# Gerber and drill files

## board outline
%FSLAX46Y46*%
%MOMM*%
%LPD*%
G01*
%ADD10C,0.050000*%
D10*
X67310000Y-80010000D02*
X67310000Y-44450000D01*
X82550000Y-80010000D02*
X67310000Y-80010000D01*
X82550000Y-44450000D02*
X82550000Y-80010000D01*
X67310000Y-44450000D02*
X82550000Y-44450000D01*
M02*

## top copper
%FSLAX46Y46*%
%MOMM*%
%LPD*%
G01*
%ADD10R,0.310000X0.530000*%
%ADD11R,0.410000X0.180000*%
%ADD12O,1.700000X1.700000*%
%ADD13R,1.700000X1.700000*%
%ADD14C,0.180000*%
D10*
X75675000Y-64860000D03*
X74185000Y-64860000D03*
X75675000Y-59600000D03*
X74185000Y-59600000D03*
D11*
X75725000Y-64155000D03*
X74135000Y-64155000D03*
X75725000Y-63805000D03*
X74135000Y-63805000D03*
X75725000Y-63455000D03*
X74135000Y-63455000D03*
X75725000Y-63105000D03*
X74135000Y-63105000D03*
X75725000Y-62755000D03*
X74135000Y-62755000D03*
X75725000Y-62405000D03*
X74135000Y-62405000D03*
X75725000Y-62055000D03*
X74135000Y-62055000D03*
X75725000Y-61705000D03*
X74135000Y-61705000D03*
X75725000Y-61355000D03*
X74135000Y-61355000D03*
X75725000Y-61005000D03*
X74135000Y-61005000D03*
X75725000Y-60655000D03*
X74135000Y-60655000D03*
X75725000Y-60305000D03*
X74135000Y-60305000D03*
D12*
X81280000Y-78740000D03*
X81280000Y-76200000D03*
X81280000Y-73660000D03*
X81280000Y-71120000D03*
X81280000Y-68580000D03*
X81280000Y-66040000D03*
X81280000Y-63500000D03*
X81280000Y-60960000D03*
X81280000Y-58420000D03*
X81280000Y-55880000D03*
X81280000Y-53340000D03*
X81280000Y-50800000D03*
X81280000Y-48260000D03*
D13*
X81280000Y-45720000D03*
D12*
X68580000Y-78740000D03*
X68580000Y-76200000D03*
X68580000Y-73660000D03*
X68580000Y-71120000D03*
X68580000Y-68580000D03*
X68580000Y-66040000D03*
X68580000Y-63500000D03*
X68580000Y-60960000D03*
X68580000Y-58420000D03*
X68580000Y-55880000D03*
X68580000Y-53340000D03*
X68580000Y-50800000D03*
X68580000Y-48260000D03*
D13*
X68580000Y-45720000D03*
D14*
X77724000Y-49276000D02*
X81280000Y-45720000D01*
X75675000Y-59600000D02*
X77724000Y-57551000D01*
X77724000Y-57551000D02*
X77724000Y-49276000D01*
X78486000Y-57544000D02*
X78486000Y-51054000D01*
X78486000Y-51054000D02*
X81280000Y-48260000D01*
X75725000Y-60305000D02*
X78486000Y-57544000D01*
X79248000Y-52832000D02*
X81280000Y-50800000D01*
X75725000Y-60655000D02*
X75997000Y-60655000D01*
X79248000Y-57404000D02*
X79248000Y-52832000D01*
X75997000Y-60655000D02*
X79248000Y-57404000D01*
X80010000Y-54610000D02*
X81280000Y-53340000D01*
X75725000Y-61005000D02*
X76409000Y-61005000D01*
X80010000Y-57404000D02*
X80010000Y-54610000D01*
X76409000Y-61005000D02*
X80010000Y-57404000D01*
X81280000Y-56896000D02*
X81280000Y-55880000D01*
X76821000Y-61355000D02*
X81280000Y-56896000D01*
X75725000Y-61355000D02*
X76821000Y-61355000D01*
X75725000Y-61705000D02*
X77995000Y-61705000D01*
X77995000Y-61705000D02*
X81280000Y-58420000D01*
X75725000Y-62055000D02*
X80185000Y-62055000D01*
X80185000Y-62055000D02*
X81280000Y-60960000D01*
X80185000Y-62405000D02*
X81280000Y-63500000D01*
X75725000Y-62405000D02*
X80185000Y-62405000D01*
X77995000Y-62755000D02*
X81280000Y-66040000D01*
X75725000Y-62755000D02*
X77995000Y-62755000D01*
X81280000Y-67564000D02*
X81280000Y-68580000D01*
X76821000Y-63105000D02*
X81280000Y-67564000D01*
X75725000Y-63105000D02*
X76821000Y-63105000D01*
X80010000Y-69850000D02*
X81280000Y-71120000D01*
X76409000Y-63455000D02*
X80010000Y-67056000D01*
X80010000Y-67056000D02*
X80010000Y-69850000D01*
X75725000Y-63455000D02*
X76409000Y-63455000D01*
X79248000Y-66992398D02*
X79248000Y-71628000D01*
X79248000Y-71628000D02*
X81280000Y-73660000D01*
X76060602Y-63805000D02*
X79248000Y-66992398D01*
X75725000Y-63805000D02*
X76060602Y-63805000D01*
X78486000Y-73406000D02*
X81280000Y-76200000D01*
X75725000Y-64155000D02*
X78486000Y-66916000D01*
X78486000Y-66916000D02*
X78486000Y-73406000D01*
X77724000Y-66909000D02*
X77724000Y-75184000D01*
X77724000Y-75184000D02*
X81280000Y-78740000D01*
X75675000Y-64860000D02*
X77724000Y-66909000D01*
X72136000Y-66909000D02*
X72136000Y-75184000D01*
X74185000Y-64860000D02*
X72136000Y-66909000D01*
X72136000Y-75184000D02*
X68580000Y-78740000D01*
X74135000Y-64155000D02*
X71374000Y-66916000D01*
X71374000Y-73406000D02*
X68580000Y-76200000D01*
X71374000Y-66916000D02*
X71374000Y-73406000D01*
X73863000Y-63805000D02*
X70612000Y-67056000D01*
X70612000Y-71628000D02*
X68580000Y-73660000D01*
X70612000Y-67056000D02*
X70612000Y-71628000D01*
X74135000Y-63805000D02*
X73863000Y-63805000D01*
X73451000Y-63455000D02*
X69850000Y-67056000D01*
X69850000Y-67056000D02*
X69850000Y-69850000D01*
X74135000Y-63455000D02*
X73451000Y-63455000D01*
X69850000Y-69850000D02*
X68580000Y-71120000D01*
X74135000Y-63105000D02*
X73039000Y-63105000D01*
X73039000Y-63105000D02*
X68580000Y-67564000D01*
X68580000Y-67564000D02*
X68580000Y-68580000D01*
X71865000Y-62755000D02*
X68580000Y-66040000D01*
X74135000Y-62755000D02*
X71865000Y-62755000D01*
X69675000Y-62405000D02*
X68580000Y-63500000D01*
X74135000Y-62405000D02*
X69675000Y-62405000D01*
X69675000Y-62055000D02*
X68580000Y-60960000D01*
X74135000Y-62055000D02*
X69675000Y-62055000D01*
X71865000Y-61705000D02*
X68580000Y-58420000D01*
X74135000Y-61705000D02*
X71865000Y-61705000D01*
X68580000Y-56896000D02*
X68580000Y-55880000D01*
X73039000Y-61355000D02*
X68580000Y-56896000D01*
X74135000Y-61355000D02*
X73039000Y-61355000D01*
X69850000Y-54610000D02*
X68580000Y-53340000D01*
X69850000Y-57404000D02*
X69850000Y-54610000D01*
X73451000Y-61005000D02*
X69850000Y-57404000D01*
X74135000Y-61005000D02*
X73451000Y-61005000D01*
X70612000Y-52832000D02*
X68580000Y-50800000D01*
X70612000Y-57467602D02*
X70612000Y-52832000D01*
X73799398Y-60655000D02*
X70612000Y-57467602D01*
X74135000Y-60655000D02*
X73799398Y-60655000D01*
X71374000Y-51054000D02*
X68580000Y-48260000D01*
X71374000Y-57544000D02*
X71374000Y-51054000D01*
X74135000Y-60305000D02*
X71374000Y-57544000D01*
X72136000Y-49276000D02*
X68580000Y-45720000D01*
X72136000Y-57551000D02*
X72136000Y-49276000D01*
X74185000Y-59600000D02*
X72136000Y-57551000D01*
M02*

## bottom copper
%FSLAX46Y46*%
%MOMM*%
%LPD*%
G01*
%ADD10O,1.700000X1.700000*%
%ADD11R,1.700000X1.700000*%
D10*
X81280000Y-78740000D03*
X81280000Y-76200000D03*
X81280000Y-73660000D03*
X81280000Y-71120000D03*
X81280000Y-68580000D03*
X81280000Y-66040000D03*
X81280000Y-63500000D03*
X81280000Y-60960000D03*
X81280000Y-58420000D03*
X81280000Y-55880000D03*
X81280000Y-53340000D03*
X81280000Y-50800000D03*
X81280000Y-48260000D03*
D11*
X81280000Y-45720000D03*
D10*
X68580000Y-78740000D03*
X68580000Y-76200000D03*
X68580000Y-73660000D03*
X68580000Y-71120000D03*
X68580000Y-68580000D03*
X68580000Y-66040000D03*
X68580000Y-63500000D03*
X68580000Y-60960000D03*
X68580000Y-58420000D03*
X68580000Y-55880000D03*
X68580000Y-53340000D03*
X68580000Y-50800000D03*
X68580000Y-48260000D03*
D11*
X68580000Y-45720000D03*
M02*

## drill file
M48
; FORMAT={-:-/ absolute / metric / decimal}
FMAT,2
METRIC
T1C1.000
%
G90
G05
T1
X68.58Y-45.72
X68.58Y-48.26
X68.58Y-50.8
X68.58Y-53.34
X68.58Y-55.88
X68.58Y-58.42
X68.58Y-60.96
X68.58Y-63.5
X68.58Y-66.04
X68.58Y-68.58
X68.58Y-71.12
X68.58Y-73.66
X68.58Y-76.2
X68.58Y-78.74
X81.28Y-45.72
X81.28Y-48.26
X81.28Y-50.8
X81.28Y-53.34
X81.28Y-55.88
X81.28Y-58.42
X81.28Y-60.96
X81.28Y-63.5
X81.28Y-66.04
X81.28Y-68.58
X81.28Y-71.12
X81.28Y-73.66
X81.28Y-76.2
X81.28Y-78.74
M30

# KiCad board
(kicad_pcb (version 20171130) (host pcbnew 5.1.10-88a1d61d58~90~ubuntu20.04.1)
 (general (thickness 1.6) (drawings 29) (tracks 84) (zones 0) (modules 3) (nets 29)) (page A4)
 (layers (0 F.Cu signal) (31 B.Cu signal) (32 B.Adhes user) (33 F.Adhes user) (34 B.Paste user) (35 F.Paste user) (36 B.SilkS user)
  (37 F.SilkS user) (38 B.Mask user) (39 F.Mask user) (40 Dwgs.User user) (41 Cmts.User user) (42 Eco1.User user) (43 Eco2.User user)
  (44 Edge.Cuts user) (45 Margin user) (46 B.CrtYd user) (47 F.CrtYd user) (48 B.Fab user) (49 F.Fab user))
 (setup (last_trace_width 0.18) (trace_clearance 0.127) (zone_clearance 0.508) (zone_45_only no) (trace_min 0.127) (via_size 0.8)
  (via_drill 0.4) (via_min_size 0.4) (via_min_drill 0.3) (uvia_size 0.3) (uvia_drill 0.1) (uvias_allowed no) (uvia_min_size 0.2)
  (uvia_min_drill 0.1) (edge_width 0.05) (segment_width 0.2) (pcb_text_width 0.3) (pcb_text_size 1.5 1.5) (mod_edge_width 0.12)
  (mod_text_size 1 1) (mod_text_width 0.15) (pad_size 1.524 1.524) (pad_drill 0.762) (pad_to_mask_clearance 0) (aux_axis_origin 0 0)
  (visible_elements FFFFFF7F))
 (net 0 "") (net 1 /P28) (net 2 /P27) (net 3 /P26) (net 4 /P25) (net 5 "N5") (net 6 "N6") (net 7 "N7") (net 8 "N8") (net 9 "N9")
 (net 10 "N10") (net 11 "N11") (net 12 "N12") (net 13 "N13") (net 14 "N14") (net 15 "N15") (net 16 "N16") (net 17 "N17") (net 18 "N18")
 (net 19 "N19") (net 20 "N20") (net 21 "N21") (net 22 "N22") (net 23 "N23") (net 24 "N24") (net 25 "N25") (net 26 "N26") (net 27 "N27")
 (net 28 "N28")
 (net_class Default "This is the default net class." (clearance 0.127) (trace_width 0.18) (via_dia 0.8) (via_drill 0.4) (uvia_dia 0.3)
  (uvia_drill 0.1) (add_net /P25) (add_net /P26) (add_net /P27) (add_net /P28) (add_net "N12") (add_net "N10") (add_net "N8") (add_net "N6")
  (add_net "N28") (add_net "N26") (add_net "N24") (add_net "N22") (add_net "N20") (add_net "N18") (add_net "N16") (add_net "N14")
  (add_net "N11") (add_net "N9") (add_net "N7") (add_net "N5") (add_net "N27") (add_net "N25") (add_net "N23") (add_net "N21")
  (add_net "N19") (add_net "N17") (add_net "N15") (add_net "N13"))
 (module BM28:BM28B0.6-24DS (layer F.Cu) (at 74.93 62.23)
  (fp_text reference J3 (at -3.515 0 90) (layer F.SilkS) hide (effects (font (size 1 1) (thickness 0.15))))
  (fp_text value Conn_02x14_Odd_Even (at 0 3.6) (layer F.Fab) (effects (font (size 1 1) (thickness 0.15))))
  (pad 28 smd rect (at 0.745 2.63) (size 0.31 0.53) (layers F.Cu F.Paste F.Mask) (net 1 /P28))
  (pad 27 smd rect (at -0.745 2.63) (size 0.31 0.53) (layers F.Cu F.Paste F.Mask) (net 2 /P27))
  (pad 26 smd rect (at 0.745 -2.63) (size 0.31 0.53) (layers F.Cu F.Paste F.Mask) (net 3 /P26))
  (pad 25 smd rect (at -0.745 -2.63) (size 0.31 0.53) (layers F.Cu F.Paste F.Mask) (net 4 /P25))
  (pad 24 smd rect (at 0.795 1.925) (size 0.41 0.18) (layers F.Cu F.Paste F.Mask) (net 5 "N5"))
  (pad 23 smd rect (at -0.795 1.925) (size 0.41 0.18) (layers F.Cu F.Paste F.Mask) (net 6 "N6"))
  (pad 22 smd rect (at 0.795 1.575) (size 0.41 0.18) (layers F.Cu F.Paste F.Mask) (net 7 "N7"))
  (pad 21 smd rect (at -0.795 1.575) (size 0.41 0.18) (layers F.Cu F.Paste F.Mask) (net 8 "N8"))
  (pad 20 smd rect (at 0.795 1.225) (size 0.41 0.18) (layers F.Cu F.Paste F.Mask) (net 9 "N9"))
  (pad 19 smd rect (at -0.795 1.225) (size 0.41 0.18) (layers F.Cu F.Paste F.Mask) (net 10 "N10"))
  (pad 18 smd rect (at 0.795 0.875) (size 0.41 0.18) (layers F.Cu F.Paste F.Mask) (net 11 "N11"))
  (pad 17 smd rect (at -0.795 0.875) (size 0.41 0.18) (layers F.Cu F.Paste F.Mask) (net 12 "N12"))
  (pad 16 smd rect (at 0.795 0.525) (size 0.41 0.18) (layers F.Cu F.Paste F.Mask) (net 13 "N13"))
  (pad 15 smd rect (at -0.795 0.525) (size 0.41 0.18) (layers F.Cu F.Paste F.Mask) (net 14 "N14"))
  (pad 14 smd rect (at 0.795 0.175) (size 0.41 0.18) (layers F.Cu F.Paste F.Mask) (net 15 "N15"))
  (pad 13 smd rect (at -0.795 0.175) (size 0.41 0.18) (layers F.Cu F.Paste F.Mask) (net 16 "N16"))
  (pad 12 smd rect (at 0.795 -0.175) (size 0.41 0.18) (layers F.Cu F.Paste F.Mask) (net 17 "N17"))
  (pad 11 smd rect (at -0.795 -0.175) (size 0.41 0.18) (layers F.Cu F.Paste F.Mask) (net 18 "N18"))
  (pad 10 smd rect (at 0.795 -0.525) (size 0.41 0.18) (layers F.Cu F.Paste F.Mask) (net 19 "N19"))
  (pad 9 smd rect (at -0.795 -0.525) (size 0.41 0.18) (layers F.Cu F.Paste F.Mask) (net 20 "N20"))
  (pad 8 smd rect (at 0.795 -0.875) (size 0.41 0.18) (layers F.Cu F.Paste F.Mask) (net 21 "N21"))
  (pad 7 smd rect (at -0.795 -0.875) (size 0.41 0.18) (layers F.Cu F.Paste F.Mask) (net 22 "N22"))
  (pad 6 smd rect (at 0.795 -1.225) (size 0.41 0.18) (layers F.Cu F.Paste F.Mask) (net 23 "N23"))
  (pad 5 smd rect (at -0.795 -1.225) (size 0.41 0.18) (layers F.Cu F.Paste F.Mask) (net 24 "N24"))
  (pad 4 smd rect (at 0.795 -1.575) (size 0.41 0.18) (layers F.Cu F.Paste F.Mask) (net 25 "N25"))
  (pad 3 smd rect (at -0.795 -1.575) (size 0.41 0.18) (layers F.Cu F.Paste F.Mask) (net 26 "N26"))
  (pad 2 smd rect (at 0.795 -1.925) (size 0.41 0.18) (layers F.Cu F.Paste F.Mask) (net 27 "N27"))
  (pad 1 smd rect (at -0.795 -1.925) (size 0.41 0.18) (layers F.Cu F.Paste F.Mask) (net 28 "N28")))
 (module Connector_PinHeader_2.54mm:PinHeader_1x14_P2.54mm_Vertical (layer B.Cu) (at 81.28 45.72 180)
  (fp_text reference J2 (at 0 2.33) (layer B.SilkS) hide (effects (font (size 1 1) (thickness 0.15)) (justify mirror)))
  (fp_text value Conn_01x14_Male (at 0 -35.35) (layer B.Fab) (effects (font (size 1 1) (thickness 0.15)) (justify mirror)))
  (pad 14 thru_hole oval (at 0 -33.02 180) (size 1.7 1.7) (drill 1) (layers *.Cu *.Mask) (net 1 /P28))
  (pad 13 thru_hole oval (at 0 -30.48 180) (size 1.7 1.7) (drill 1) (layers *.Cu *.Mask) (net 5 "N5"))
  (pad 12 thru_hole oval (at 0 -27.94 180) (size 1.7 1.7) (drill 1) (layers *.Cu *.Mask) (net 7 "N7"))
  (pad 11 thru_hole oval (at 0 -25.4 180) (size 1.7 1.7) (drill 1) (layers *.Cu *.Mask) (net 9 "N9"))
  (pad 10 thru_hole oval (at 0 -22.86 180) (size 1.7 1.7) (drill 1) (layers *.Cu *.Mask) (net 11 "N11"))
  (pad 9 thru_hole oval (at 0 -20.32 180) (size 1.7 1.7) (drill 1) (layers *.Cu *.Mask) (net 13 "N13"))
  (pad 8 thru_hole oval (at 0 -17.78 180) (size 1.7 1.7) (drill 1) (layers *.Cu *.Mask) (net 15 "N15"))
  (pad 7 thru_hole oval (at 0 -15.24 180) (size 1.7 1.7) (drill 1) (layers *.Cu *.Mask) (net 17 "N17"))
  (pad 6 thru_hole oval (at 0 -12.7 180) (size 1.7 1.7) (drill 1) (layers *.Cu *.Mask) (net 19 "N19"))
  (pad 5 thru_hole oval (at 0 -10.16 180) (size 1.7 1.7) (drill 1) (layers *.Cu *.Mask) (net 21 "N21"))
  (pad 4 thru_hole oval (at 0 -7.62 180) (size 1.7 1.7) (drill 1) (layers *.Cu *.Mask) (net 23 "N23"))
  (pad 3 thru_hole oval (at 0 -5.08 180) (size 1.7 1.7) (drill 1) (layers *.Cu *.Mask) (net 25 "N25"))
  (pad 2 thru_hole oval (at 0 -2.54 180) (size 1.7 1.7) (drill 1) (layers *.Cu *.Mask) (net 27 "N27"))
  (pad 1 thru_hole rect (at 0 0 180) (size 1.7 1.7) (drill 1) (layers *.Cu *.Mask) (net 3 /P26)))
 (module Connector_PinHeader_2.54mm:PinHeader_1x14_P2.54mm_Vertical (layer B.Cu) (at 68.58 45.72 180)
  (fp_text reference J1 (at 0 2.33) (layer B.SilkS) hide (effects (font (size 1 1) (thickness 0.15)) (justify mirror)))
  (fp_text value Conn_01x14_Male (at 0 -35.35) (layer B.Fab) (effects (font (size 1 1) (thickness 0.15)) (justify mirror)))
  (pad 14 thru_hole oval (at 0 -33.02 180) (size 1.7 1.7) (drill 1) (layers *.Cu *.Mask) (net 2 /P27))
  (pad 13 thru_hole oval (at 0 -30.48 180) (size 1.7 1.7) (drill 1) (layers *.Cu *.Mask) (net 6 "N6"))
  (pad 12 thru_hole oval (at 0 -27.94 180) (size 1.7 1.7) (drill 1) (layers *.Cu *.Mask) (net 8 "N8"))
  (pad 11 thru_hole oval (at 0 -25.4 180) (size 1.7 1.7) (drill 1) (layers *.Cu *.Mask) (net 10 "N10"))
  (pad 10 thru_hole oval (at 0 -22.86 180) (size 1.7 1.7) (drill 1) (layers *.Cu *.Mask) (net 12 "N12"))
  (pad 9 thru_hole oval (at 0 -20.32 180) (size 1.7 1.7) (drill 1) (layers *.Cu *.Mask) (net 14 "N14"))
  (pad 8 thru_hole oval (at 0 -17.78 180) (size 1.7 1.7) (drill 1) (layers *.Cu *.Mask) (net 16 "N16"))
  (pad 7 thru_hole oval (at 0 -15.24 180) (size 1.7 1.7) (drill 1) (layers *.Cu *.Mask) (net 18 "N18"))
  (pad 6 thru_hole oval (at 0 -12.7 180) (size 1.7 1.7) (drill 1) (layers *.Cu *.Mask) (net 20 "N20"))
  (pad 5 thru_hole oval (at 0 -10.16 180) (size 1.7 1.7) (drill 1) (layers *.Cu *.Mask) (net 22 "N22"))
  (pad 4 thru_hole oval (at 0 -7.62 180) (size 1.7 1.7) (drill 1) (layers *.Cu *.Mask) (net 24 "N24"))
  (pad 3 thru_hole oval (at 0 -5.08 180) (size 1.7 1.7) (drill 1) (layers *.Cu *.Mask) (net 26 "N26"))
  (pad 2 thru_hole oval (at 0 -2.54 180) (size 1.7 1.7) (drill 1) (layers *.Cu *.Mask) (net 28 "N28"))
  (pad 1 thru_hole rect (at 0 0 180) (size 1.7 1.7) (drill 1) (layers *.Cu *.Mask) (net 4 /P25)))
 (gr_line (start 67.31 80.01) (end 67.31 44.45) (layer Edge.Cuts) (width 0.05))
 (gr_line (start 82.55 80.01) (end 67.31 80.01) (layer Edge.Cuts) (width 0.05))
 (gr_line (start 82.55 44.45) (end 82.55 80.01) (layer Edge.Cuts) (width 0.05))
 (gr_line (start 67.31 44.45) (end 82.55 44.45) (layer Edge.Cuts) (width 0.05))
 (segment (start 77.724 49.276) (end 81.28 45.72) (width 0.18) (layer F.Cu) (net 3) (status 20))
 (segment (start 75.675 59.6) (end 77.724 57.551) (width 0.18) (layer F.Cu) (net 3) (status 10))
 (segment (start 77.724 57.551) (end 77.724 49.276) (width 0.18) (layer F.Cu) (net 3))
 (segment (start 78.486 57.544) (end 78.486 51.054) (width 0.18) (layer F.Cu) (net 27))
 (segment (start 78.486 51.054) (end 81.28 48.26) (width 0.18) (layer F.Cu) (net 27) (status 20))
 (segment (start 75.725 60.305) (end 78.486 57.544) (width 0.18) (layer F.Cu) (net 27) (status 10))
 (segment (start 79.248 52.832) (end 81.28 50.8) (width 0.18) (layer F.Cu) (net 25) (status 20))
 (segment (start 75.725 60.655) (end 75.997 60.655) (width 0.18) (layer F.Cu) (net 25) (status 10))
 (segment (start 79.248 57.404) (end 79.248 52.832) (width 0.18) (layer F.Cu) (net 25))
 (segment (start 75.997 60.655) (end 79.248 57.404) (width 0.18) (layer F.Cu) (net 25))
 (segment (start 80.01 54.61) (end 81.28 53.34) (width 0.18) (layer F.Cu) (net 23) (status 20))
 (segment (start 75.725 61.005) (end 76.409 61.005) (width 0.18) (layer F.Cu) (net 23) (status 10))
 (segment (start 80.01 57.404) (end 80.01 54.61) (width 0.18) (layer F.Cu) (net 23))
 (segment (start 76.409 61.005) (end 80.01 57.404) (width 0.18) (layer F.Cu) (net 23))
 (segment (start 81.28 56.896) (end 81.28 55.88) (width 0.18) (layer F.Cu) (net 21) (status 20))
 (segment (start 76.821 61.355) (end 81.28 56.896) (width 0.18) (layer F.Cu) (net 21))
 (segment (start 75.725 61.355) (end 76.821 61.355) (width 0.18) (layer F.Cu) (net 21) (status 10))
 (segment (start 75.725 61.705) (end 77.995 61.705) (width 0.18) (layer F.Cu) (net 19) (status 10))
 (segment (start 77.995 61.705) (end 81.28 58.42) (width 0.18) (layer F.Cu) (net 19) (status 20))
 (segment (start 75.725 62.055) (end 80.185 62.055) (width 0.18) (layer F.Cu) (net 17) (status 10))
 (segment (start 80.185 62.055) (end 81.28 60.96) (width 0.18) (layer F.Cu) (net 17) (status 20))
 (segment (start 80.185 62.405) (end 81.28 63.5) (width 0.18) (layer F.Cu) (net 15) (status 20))
 (segment (start 75.725 62.405) (end 80.185 62.405) (width 0.18) (layer F.Cu) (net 15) (status 10))
 (segment (start 77.995 62.755) (end 81.28 66.04) (width 0.18) (layer F.Cu) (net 13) (status 20))
 (segment (start 75.725 62.755) (end 77.995 62.755) (width 0.18) (layer F.Cu) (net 13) (status 10))
 (segment (start 81.28 67.564) (end 81.28 68.58) (width 0.18) (layer F.Cu) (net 11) (status 20))
 (segment (start 76.821 63.105) (end 81.28 67.564) (width 0.18) (layer F.Cu) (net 11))
 (segment (start 75.725 63.105) (end 76.821 63.105) (width 0.18) (layer F.Cu) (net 11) (status 10))
 (segment (start 80.01 69.85) (end 81.28 71.12) (width 0.18) (layer F.Cu) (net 9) (status 20))
 (segment (start 76.409 63.455) (end 80.01 67.056) (width 0.18) (layer F.Cu) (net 9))
 (segment (start 80.01 67.056) (end 80.01 69.85) (width 0.18) (layer F.Cu) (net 9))
 (segment (start 75.725 63.455) (end 76.409 63.455) (width 0.18) (layer F.Cu) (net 9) (status 10))
 (segment (start 79.248 66.992398) (end 79.248 71.628) (width 0.18) (layer F.Cu) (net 7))
 (segment (start 79.248 71.628) (end 81.28 73.66) (width 0.18) (layer F.Cu) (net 7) (status 20))
 (segment (start 76.060602 63.805) (end 79.248 66.992398) (width 0.18) (layer F.Cu) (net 7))
 (segment (start 75.725 63.805) (end 76.060602 63.805) (width 0.18) (layer F.Cu) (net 7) (status 10))
 (segment (start 78.486 73.406) (end 81.28 76.2) (width 0.18) (layer F.Cu) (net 5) (status 20))
 (segment (start 75.725 64.155) (end 78.486 66.916) (width 0.18) (layer F.Cu) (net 5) (status 10))
 (segment (start 78.486 66.916) (end 78.486 73.406) (width 0.18) (layer F.Cu) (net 5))
 (segment (start 77.724 66.909) (end 77.724 75.184) (width 0.18) (layer F.Cu) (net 1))
 (segment (start 77.724 75.184) (end 81.28 78.74) (width 0.18) (layer F.Cu) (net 1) (status 20))
 (segment (start 75.675 64.86) (end 77.724 66.909) (width 0.18) (layer F.Cu) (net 1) (status 10))
 (segment (start 72.136 66.909) (end 72.136 75.184) (width 0.18) (layer F.Cu) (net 2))
 (segment (start 74.185 64.86) (end 72.136 66.909) (width 0.18) (layer F.Cu) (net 2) (status 10))
 (segment (start 72.136 75.184) (end 68.58 78.74) (width 0.18) (layer F.Cu) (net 2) (status 20))
 (segment (start 74.135 64.155) (end 71.374 66.916) (width 0.18) (layer F.Cu) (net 6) (status 10))
 (segment (start 71.374 73.406) (end 68.58 76.2) (width 0.18) (layer F.Cu) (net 6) (status 20))
 (segment (start 71.374 66.916) (end 71.374 73.406) (width 0.18) (layer F.Cu) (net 6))
 (segment (start 73.863 63.805) (end 70.612 67.056) (width 0.18) (layer F.Cu) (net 8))
 (segment (start 70.612 71.628) (end 68.58 73.66) (width 0.18) (layer F.Cu) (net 8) (status 20))
 (segment (start 70.612 67.056) (end 70.612 71.628) (width 0.18) (layer F.Cu) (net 8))
 (segment (start 74.135 63.805) (end 73.863 63.805) (width 0.18) (layer F.Cu) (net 8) (status 10))
 (segment (start 73.451 63.455) (end 69.85 67.056) (width 0.18) (layer F.Cu) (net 10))
 (segment (start 69.85 67.056) (end 69.85 69.85) (width 0.18) (layer F.Cu) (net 10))
 (segment (start 74.135 63.455) (end 73.451 63.455) (width 0.18) (layer F.Cu) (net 10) (status 10))
 (segment (start 69.85 69.85) (end 68.58 71.12) (width 0.18) (layer F.Cu) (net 10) (status 20))
 (segment (start 74.135 63.105) (end 73.039 63.105) (width 0.18) (layer F.Cu) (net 12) (status 10))
 (segment (start 73.039 63.105) (end 68.58 67.564) (width 0.18) (layer F.Cu) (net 12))
 (segment (start 68.58 67.564) (end 68.58 68.58) (width 0.18) (layer F.Cu) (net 12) (status 20))
 (segment (start 71.865 62.755) (end 68.58 66.04) (width 0.18) (layer F.Cu) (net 14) (status 20))
 (segment (start 74.135 62.755) (end 71.865 62.755) (width 0.18) (layer F.Cu) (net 14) (status 10))
 (segment (start 69.675 62.405) (end 68.58 63.5) (width 0.18) (layer F.Cu) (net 16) (status 20))
 (segment (start 74.135 62.405) (end 69.675 62.405) (width 0.18) (layer F.Cu) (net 16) (status 10))
 (segment (start 69.675 62.055) (end 68.58 60.96) (width 0.18) (layer F.Cu) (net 18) (status 20))
 (segment (start 74.135 62.055) (end 69.675 62.055) (width 0.18) (layer F.Cu) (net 18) (status 10))
 (segment (start 71.865 61.705) (end 68.58 58.42) (width 0.18) (layer F.Cu) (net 20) (status 20))
 (segment (start 74.135 61.705) (end 71.865 61.705) (width 0.18) (layer F.Cu) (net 20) (status 10))
 (segment (start 68.58 56.896) (end 68.58 55.88) (width 0.18) (layer F.Cu) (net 22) (status 20))
 (segment (start 73.039 61.355) (end 68.58 56.896) (width 0.18) (layer F.Cu) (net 22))
 (segment (start 74.135 61.355) (end 73.039 61.355) (width 0.18) (layer F.Cu) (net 22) (status 10))
 (segment (start 69.85 54.61) (end 68.58 53.34) (width 0.18) (layer F.Cu) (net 24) (status 20))
 (segment (start 69.85 57.404) (end 69.85 54.61) (width 0.18) (layer F.Cu) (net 24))
 (segment (start 73.451 61.005) (end 69.85 57.404) (width 0.18) (layer F.Cu) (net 24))
 (segment (start 74.135 61.005) (end 73.451 61.005) (width 0.18) (layer F.Cu) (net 24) (status 10))
 (segment (start 70.612 52.832) (end 68.58 50.8) (width 0.18) (layer F.Cu) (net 26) (status 20))
 (segment (start 70.612 57.467602) (end 70.612 52.832) (width 0.18) (layer F.Cu) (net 26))
 (segment (start 73.799398 60.655) (end 70.612 57.467602) (width 0.18) (layer F.Cu) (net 26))
 (segment (start 74.135 60.655) (end 73.799398 60.655) (width 0.18) (layer F.Cu) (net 26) (status 10))
 (segment (start 71.374 51.054) (end 68.58 48.26) (width 0.18) (layer F.Cu) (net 28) (status 20))
 (segment (start 71.374 57.544) (end 71.374 51.054) (width 0.18) (layer F.Cu) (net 28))
 (segment (start 74.135 60.305) (end 71.374 57.544) (width 0.18) (layer F.Cu) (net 28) (status 10))
 (segment (start 72.136 49.276) (end 68.58 45.72) (width 0.18) (layer F.Cu) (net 4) (status 20))
 (segment (start 72.136 57.551) (end 72.136 49.276) (width 0.18) (layer F.Cu) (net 4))
 (segment (start 74.185 59.6) (end 72.136 57.551) (width 0.18) (layer F.Cu) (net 4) (status 10)))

